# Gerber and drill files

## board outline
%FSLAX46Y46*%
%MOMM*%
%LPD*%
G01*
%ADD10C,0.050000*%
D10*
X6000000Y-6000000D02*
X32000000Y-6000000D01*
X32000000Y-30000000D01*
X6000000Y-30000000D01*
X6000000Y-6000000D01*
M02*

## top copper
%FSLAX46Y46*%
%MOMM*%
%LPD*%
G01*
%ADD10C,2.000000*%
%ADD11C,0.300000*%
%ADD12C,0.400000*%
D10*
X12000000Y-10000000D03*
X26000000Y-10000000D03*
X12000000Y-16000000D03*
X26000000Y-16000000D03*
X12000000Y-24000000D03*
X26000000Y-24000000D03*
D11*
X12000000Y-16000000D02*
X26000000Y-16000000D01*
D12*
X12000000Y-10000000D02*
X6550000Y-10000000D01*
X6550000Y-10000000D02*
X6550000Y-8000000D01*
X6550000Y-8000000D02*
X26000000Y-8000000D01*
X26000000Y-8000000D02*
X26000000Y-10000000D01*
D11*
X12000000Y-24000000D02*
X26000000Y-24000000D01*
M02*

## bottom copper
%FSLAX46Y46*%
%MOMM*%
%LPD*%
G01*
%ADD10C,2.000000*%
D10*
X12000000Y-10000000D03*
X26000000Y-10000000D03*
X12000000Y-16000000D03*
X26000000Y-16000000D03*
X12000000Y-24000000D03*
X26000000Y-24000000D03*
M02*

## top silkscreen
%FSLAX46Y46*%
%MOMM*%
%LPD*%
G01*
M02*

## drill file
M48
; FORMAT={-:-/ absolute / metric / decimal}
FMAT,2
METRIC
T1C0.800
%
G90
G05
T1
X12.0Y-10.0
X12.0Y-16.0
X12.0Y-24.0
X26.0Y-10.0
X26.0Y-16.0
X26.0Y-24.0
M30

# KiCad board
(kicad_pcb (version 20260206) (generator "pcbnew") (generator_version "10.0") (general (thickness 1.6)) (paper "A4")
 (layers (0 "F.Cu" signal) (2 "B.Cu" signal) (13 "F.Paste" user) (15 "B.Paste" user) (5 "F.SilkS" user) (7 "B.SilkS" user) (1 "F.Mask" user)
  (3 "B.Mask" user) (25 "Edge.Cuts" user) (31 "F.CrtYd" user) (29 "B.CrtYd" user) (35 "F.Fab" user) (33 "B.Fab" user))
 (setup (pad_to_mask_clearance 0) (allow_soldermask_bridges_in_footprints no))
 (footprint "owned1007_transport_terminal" (layer "F.Cu") (at 12 10)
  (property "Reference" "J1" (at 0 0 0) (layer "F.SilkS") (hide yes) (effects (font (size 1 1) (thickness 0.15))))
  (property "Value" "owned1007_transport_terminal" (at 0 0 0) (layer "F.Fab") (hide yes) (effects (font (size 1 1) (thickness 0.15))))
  (pad "1" thru_hole circle (at 0 0) (size 2 2) (drill 0.8) (layers "*.Cu" "*.Mask") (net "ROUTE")))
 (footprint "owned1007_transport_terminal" (layer "F.Cu") (at 26 10)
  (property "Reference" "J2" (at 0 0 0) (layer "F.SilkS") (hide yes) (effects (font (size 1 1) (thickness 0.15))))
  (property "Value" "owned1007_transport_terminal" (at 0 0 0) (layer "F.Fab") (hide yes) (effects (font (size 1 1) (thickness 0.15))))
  (pad "1" thru_hole circle (at 0 0) (size 2 2) (drill 0.8) (layers "*.Cu" "*.Mask") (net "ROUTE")))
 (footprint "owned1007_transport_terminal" (layer "F.Cu") (at 12 16)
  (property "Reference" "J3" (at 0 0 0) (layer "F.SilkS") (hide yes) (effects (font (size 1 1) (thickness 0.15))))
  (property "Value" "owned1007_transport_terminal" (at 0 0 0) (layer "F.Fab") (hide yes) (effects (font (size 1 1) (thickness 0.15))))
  (pad "1" thru_hole circle (at 0 0) (size 2 2) (drill 0.8) (layers "*.Cu" "*.Mask") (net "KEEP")))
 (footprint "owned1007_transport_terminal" (layer "F.Cu") (at 26 16)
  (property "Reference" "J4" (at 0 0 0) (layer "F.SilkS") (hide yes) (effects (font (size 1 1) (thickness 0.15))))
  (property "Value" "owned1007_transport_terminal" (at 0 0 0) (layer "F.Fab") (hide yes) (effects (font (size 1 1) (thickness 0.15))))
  (pad "1" thru_hole circle (at 0 0) (size 2 2) (drill 0.8) (layers "*.Cu" "*.Mask") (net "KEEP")))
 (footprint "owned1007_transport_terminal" (layer "F.Cu") (at 12 24)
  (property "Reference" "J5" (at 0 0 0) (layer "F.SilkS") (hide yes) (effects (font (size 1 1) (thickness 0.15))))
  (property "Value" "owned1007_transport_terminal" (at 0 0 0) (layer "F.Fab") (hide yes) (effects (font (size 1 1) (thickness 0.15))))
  (pad "1" thru_hole circle (at 0 0) (size 2 2) (drill 0.8) (layers "*.Cu" "*.Mask") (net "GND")))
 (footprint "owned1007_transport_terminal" (layer "F.Cu") (at 26 24)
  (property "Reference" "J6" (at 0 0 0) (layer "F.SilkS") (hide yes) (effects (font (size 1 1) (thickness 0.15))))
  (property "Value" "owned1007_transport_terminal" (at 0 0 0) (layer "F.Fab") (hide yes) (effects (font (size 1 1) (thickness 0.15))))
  (pad "1" thru_hole circle (at 0 0) (size 2 2) (drill 0.8) (layers "*.Cu" "*.Mask") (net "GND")))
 (gr_rect (start 6 6) (end 32 30) (stroke (width 0.05) (type default)) (fill none) (layer "Edge.Cuts"))
 (segment (start 12 16) (end 26 16) (width 0.3) (layer "F.Cu") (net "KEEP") (locked yes))
 (segment (start 12 10) (end 6.55 10) (width 0.4) (layer "F.Cu") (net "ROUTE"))
 (segment (start 6.55 10) (end 6.55 8) (width 0.4) (layer "F.Cu") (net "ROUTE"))
 (segment (start 6.55 8) (end 26 8) (width 0.4) (layer "F.Cu") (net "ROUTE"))
 (segment (start 26 8) (end 26 10) (width 0.4) (layer "F.Cu") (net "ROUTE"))
 (segment (start 12 24) (end 26 24) (width 0.3) (layer "F.Cu") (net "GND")))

